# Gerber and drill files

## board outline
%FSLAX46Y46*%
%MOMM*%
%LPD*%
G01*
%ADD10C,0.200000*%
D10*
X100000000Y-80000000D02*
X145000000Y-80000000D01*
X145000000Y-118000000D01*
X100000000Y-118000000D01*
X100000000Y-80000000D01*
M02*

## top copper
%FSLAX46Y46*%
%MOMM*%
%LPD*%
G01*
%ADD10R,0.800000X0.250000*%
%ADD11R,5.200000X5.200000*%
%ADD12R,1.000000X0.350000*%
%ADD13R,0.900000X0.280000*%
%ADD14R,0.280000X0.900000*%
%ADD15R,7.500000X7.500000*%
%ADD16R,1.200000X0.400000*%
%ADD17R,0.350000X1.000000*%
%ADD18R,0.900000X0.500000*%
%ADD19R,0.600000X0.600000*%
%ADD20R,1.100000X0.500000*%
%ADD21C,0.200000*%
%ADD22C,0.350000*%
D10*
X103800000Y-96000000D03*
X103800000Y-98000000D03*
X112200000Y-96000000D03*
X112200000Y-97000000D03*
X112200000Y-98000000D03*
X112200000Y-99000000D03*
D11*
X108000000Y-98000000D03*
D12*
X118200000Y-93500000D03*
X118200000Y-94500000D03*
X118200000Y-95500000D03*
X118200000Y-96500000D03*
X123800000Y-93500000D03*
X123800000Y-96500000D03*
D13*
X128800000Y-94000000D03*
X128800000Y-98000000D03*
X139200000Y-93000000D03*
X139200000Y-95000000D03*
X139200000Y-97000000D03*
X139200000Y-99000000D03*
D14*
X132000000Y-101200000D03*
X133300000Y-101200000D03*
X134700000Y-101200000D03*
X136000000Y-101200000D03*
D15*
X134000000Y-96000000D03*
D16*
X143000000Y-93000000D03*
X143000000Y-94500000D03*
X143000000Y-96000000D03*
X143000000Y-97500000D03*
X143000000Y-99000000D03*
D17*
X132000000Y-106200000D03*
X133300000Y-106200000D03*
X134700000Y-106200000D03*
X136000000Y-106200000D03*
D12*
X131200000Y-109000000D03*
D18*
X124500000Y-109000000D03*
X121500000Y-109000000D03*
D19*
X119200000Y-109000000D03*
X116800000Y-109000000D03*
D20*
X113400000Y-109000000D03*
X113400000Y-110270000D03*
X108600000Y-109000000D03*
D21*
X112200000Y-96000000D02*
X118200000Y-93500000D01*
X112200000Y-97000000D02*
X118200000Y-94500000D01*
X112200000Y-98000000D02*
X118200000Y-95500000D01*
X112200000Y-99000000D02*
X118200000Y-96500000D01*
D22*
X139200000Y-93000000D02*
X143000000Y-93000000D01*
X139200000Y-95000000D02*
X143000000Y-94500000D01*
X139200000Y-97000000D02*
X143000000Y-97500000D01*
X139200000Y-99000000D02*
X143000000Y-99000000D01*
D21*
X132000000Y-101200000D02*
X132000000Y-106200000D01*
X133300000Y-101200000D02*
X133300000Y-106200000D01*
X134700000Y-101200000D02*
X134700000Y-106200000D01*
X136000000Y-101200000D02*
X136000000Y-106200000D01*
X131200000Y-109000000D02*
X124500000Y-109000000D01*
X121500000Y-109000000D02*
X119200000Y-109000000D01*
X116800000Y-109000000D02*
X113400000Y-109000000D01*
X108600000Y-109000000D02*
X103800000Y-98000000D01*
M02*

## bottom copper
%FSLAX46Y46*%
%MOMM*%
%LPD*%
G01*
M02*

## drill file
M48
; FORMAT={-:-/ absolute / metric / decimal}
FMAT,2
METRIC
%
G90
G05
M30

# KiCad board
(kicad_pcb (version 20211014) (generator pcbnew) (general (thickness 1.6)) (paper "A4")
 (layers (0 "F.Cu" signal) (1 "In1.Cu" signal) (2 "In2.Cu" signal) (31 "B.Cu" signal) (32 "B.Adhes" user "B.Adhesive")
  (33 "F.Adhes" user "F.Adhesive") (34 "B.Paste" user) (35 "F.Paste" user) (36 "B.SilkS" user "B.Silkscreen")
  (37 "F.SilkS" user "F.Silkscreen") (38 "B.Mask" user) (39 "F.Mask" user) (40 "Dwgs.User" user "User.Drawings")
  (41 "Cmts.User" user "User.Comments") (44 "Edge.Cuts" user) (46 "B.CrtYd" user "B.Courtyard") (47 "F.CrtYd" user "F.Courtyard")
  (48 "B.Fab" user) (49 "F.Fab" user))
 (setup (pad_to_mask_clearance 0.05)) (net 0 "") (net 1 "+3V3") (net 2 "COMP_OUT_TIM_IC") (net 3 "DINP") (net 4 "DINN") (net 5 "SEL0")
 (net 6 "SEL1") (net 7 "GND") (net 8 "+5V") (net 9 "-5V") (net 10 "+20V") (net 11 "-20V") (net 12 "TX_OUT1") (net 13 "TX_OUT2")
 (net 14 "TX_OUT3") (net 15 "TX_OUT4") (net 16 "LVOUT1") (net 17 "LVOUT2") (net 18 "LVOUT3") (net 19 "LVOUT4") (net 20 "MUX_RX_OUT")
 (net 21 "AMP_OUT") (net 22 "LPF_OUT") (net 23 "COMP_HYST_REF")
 (gr_rect (start 100 80) (end 145 118) (layer "Edge.Cuts") (width 0.2))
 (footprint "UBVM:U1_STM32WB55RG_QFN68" (layer "F.Cu") (at 108 98)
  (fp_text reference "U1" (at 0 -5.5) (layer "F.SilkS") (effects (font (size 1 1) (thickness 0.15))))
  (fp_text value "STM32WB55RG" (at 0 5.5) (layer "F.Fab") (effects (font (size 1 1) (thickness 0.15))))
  (pad "1" smd rect (at -4.2 -2.0) (size 0.8 0.25) (layers "F.Cu" "F.Paste" "F.Mask") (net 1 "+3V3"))
  (pad "2" smd rect (at -4.2 0.0) (size 0.8 0.25) (layers "F.Cu" "F.Paste" "F.Mask") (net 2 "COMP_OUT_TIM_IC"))
  (pad "3" smd rect (at 4.2 -2.0) (size 0.8 0.25) (layers "F.Cu" "F.Paste" "F.Mask") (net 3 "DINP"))
  (pad "4" smd rect (at 4.2 -1.0) (size 0.8 0.25) (layers "F.Cu" "F.Paste" "F.Mask") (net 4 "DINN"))
  (pad "5" smd rect (at 4.2 0.0) (size 0.8 0.25) (layers "F.Cu" "F.Paste" "F.Mask") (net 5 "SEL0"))
  (pad "6" smd rect (at 4.2 1.0) (size 0.8 0.25) (layers "F.Cu" "F.Paste" "F.Mask") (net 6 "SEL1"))
  (pad "69" smd rect (at 0 0) (size 5.2 5.2) (layers "F.Cu" "F.Paste" "F.Mask") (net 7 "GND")))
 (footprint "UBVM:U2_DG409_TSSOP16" (layer "F.Cu") (at 121 95)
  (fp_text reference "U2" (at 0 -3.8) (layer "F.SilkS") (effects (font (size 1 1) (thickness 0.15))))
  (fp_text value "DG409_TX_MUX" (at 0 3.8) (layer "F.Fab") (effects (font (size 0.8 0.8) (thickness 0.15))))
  (pad "1" smd rect (at -2.8 -1.5) (size 1.0 0.35) (layers "F.Cu" "F.Paste" "F.Mask") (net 3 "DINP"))
  (pad "2" smd rect (at -2.8 -0.5) (size 1.0 0.35) (layers "F.Cu" "F.Paste" "F.Mask") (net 4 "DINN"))
  (pad "3" smd rect (at -2.8 0.5) (size 1.0 0.35) (layers "F.Cu" "F.Paste" "F.Mask") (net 5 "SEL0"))
  (pad "4" smd rect (at -2.8 1.5) (size 1.0 0.35) (layers "F.Cu" "F.Paste" "F.Mask") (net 6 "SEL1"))
  (pad "13" smd rect (at 2.8 -1.5) (size 1.0 0.35) (layers "F.Cu" "F.Paste" "F.Mask") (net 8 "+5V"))
  (pad "14" smd rect (at 2.8 1.5) (size 1.0 0.35) (layers "F.Cu" "F.Paste" "F.Mask") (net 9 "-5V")))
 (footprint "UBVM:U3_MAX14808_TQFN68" (layer "F.Cu") (at 134 96)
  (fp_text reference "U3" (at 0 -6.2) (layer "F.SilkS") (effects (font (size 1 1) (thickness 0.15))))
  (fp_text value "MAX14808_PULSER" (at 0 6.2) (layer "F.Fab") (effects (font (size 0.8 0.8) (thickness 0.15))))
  (pad "1" smd rect (at -5.2 -2.0) (size 0.9 0.28) (layers "F.Cu" "F.Paste" "F.Mask") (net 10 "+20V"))
  (pad "2" smd rect (at -5.2 2.0) (size 0.9 0.28) (layers "F.Cu" "F.Paste" "F.Mask") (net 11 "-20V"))
  (pad "20" smd rect (at 5.2 -3.0) (size 0.9 0.28) (layers "F.Cu" "F.Paste" "F.Mask") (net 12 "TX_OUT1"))
  (pad "21" smd rect (at 5.2 -1.0) (size 0.9 0.28) (layers "F.Cu" "F.Paste" "F.Mask") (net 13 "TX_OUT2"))
  (pad "22" smd rect (at 5.2 1.0) (size 0.9 0.28) (layers "F.Cu" "F.Paste" "F.Mask") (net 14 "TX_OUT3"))
  (pad "23" smd rect (at 5.2 3.0) (size 0.9 0.28) (layers "F.Cu" "F.Paste" "F.Mask") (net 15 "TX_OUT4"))
  (pad "40" smd rect (at -2.0 5.2) (size 0.28 0.9) (layers "F.Cu" "F.Paste" "F.Mask") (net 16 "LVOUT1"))
  (pad "41" smd rect (at -0.7 5.2) (size 0.28 0.9) (layers "F.Cu" "F.Paste" "F.Mask") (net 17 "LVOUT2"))
  (pad "42" smd rect (at 0.7 5.2) (size 0.28 0.9) (layers "F.Cu" "F.Paste" "F.Mask") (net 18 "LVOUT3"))
  (pad "43" smd rect (at 2.0 5.2) (size 0.28 0.9) (layers "F.Cu" "F.Paste" "F.Mask") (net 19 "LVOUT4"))
  (pad "69" smd rect (at 0 0) (size 7.5 7.5) (layers "F.Cu" "F.Paste" "F.Mask") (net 7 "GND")))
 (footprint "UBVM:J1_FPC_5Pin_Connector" (layer "F.Cu") (at 143 96)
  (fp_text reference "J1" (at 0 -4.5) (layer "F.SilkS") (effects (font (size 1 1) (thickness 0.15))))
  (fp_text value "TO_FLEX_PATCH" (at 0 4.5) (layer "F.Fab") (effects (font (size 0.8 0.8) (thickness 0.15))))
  (pad "1" smd rect (at 0 -3.0) (size 1.2 0.4) (layers "F.Cu" "F.Paste" "F.Mask") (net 12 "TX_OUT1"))
  (pad "2" smd rect (at 0 -1.5) (size 1.2 0.4) (layers "F.Cu" "F.Paste" "F.Mask") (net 13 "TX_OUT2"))
  (pad "3" smd rect (at 0 0.0) (size 1.2 0.4) (layers "F.Cu" "F.Paste" "F.Mask") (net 7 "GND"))
  (pad "4" smd rect (at 0 1.5) (size 1.2 0.4) (layers "F.Cu" "F.Paste" "F.Mask") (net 14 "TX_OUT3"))
  (pad "5" smd rect (at 0 3.0) (size 1.2 0.4) (layers "F.Cu" "F.Paste" "F.Mask") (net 15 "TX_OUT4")))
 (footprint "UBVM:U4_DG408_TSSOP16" (layer "F.Cu") (at 134 109)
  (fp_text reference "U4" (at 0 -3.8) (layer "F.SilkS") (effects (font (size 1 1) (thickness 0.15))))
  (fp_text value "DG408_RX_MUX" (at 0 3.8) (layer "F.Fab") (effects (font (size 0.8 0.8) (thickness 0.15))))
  (pad "1" smd rect (at -2.0 -2.8) (size 0.35 1.0) (layers "F.Cu" "F.Paste" "F.Mask") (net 16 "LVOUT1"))
  (pad "2" smd rect (at -0.7 -2.8) (size 0.35 1.0) (layers "F.Cu" "F.Paste" "F.Mask") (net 17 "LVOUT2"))
  (pad "3" smd rect (at 0.7 -2.8) (size 0.35 1.0) (layers "F.Cu" "F.Paste" "F.Mask") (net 18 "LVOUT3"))
  (pad "4" smd rect (at 2.0 -2.8) (size 0.35 1.0) (layers "F.Cu" "F.Paste" "F.Mask") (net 19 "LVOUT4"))
  (pad "8" smd rect (at -2.8 0.0) (size 1.0 0.35) (layers "F.Cu" "F.Paste" "F.Mask") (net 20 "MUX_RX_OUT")))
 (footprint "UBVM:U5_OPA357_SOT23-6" (layer "F.Cu") (at 123 109)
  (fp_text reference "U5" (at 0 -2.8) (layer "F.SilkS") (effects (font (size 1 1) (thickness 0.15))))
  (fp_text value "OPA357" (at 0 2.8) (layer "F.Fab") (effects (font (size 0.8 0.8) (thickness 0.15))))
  (pad "3" smd rect (at 1.5 0.0) (size 0.9 0.5) (layers "F.Cu" "F.Paste" "F.Mask") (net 20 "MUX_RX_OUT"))
  (pad "1" smd rect (at -1.5 0.0) (size 0.9 0.5) (layers "F.Cu" "F.Paste" "F.Mask") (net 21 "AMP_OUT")))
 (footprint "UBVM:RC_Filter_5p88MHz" (layer "F.Cu") (at 118 109)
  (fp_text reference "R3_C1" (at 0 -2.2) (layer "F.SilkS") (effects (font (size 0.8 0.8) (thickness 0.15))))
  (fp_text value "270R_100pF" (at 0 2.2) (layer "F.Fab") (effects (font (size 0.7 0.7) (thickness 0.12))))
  (pad "1" smd rect (at 1.2 0.0) (size 0.6 0.6) (layers "F.Cu" "F.Paste" "F.Mask") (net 21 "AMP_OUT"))
  (pad "2" smd rect (at -1.2 0.0) (size 0.6 0.6) (layers "F.Cu" "F.Paste" "F.Mask") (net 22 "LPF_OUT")))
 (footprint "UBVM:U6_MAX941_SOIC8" (layer "F.Cu") (at 111 109)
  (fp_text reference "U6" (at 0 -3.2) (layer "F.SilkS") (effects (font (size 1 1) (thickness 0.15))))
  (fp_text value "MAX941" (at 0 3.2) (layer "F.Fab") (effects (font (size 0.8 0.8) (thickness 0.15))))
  (pad "2" smd rect (at 2.4 0.0) (size 1.1 0.5) (layers "F.Cu" "F.Paste" "F.Mask") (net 22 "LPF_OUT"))
  (pad "3" smd rect (at 2.4 1.27) (size 1.1 0.5) (layers "F.Cu" "F.Paste" "F.Mask") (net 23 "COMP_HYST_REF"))
  (pad "7" smd rect (at -2.4 0.0) (size 1.1 0.5) (layers "F.Cu" "F.Paste" "F.Mask") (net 2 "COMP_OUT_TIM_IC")))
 (segment (start 112.2 96.0) (end 118.2 93.5) (width 0.2) (layer "F.Cu") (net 3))
 (segment (start 112.2 97.0) (end 118.2 94.5) (width 0.2) (layer "F.Cu") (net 4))
 (segment (start 112.2 98.0) (end 118.2 95.5) (width 0.2) (layer "F.Cu") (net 5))
 (segment (start 112.2 99.0) (end 118.2 96.5) (width 0.2) (layer "F.Cu") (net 6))
 (segment (start 139.2 93.0) (end 143.0 93.0) (width 0.35) (layer "F.Cu") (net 12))
 (segment (start 139.2 95.0) (end 143.0 94.5) (width 0.35) (layer "F.Cu") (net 13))
 (segment (start 139.2 97.0) (end 143.0 97.5) (width 0.35) (layer "F.Cu") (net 14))
 (segment (start 139.2 99.0) (end 143.0 99.0) (width 0.35) (layer "F.Cu") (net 15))
 (segment (start 132.0 101.2) (end 132.0 106.2) (width 0.2) (layer "F.Cu") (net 16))
 (segment (start 133.3 101.2) (end 133.3 106.2) (width 0.2) (layer "F.Cu") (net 17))
 (segment (start 134.7 101.2) (end 134.7 106.2) (width 0.2) (layer "F.Cu") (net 18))
 (segment (start 136.0 101.2) (end 136.0 106.2) (width 0.2) (layer "F.Cu") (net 19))
 (segment (start 131.2 109.0) (end 124.5 109.0) (width 0.2) (layer "F.Cu") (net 20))
 (segment (start 121.5 109.0) (end 119.2 109.0) (width 0.2) (layer "F.Cu") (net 21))
 (segment (start 116.8 109.0) (end 113.4 109.0) (width 0.2) (layer "F.Cu") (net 22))
 (segment (start 108.6 109.0) (end 103.8 98.0) (width 0.2) (layer "F.Cu") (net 2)))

